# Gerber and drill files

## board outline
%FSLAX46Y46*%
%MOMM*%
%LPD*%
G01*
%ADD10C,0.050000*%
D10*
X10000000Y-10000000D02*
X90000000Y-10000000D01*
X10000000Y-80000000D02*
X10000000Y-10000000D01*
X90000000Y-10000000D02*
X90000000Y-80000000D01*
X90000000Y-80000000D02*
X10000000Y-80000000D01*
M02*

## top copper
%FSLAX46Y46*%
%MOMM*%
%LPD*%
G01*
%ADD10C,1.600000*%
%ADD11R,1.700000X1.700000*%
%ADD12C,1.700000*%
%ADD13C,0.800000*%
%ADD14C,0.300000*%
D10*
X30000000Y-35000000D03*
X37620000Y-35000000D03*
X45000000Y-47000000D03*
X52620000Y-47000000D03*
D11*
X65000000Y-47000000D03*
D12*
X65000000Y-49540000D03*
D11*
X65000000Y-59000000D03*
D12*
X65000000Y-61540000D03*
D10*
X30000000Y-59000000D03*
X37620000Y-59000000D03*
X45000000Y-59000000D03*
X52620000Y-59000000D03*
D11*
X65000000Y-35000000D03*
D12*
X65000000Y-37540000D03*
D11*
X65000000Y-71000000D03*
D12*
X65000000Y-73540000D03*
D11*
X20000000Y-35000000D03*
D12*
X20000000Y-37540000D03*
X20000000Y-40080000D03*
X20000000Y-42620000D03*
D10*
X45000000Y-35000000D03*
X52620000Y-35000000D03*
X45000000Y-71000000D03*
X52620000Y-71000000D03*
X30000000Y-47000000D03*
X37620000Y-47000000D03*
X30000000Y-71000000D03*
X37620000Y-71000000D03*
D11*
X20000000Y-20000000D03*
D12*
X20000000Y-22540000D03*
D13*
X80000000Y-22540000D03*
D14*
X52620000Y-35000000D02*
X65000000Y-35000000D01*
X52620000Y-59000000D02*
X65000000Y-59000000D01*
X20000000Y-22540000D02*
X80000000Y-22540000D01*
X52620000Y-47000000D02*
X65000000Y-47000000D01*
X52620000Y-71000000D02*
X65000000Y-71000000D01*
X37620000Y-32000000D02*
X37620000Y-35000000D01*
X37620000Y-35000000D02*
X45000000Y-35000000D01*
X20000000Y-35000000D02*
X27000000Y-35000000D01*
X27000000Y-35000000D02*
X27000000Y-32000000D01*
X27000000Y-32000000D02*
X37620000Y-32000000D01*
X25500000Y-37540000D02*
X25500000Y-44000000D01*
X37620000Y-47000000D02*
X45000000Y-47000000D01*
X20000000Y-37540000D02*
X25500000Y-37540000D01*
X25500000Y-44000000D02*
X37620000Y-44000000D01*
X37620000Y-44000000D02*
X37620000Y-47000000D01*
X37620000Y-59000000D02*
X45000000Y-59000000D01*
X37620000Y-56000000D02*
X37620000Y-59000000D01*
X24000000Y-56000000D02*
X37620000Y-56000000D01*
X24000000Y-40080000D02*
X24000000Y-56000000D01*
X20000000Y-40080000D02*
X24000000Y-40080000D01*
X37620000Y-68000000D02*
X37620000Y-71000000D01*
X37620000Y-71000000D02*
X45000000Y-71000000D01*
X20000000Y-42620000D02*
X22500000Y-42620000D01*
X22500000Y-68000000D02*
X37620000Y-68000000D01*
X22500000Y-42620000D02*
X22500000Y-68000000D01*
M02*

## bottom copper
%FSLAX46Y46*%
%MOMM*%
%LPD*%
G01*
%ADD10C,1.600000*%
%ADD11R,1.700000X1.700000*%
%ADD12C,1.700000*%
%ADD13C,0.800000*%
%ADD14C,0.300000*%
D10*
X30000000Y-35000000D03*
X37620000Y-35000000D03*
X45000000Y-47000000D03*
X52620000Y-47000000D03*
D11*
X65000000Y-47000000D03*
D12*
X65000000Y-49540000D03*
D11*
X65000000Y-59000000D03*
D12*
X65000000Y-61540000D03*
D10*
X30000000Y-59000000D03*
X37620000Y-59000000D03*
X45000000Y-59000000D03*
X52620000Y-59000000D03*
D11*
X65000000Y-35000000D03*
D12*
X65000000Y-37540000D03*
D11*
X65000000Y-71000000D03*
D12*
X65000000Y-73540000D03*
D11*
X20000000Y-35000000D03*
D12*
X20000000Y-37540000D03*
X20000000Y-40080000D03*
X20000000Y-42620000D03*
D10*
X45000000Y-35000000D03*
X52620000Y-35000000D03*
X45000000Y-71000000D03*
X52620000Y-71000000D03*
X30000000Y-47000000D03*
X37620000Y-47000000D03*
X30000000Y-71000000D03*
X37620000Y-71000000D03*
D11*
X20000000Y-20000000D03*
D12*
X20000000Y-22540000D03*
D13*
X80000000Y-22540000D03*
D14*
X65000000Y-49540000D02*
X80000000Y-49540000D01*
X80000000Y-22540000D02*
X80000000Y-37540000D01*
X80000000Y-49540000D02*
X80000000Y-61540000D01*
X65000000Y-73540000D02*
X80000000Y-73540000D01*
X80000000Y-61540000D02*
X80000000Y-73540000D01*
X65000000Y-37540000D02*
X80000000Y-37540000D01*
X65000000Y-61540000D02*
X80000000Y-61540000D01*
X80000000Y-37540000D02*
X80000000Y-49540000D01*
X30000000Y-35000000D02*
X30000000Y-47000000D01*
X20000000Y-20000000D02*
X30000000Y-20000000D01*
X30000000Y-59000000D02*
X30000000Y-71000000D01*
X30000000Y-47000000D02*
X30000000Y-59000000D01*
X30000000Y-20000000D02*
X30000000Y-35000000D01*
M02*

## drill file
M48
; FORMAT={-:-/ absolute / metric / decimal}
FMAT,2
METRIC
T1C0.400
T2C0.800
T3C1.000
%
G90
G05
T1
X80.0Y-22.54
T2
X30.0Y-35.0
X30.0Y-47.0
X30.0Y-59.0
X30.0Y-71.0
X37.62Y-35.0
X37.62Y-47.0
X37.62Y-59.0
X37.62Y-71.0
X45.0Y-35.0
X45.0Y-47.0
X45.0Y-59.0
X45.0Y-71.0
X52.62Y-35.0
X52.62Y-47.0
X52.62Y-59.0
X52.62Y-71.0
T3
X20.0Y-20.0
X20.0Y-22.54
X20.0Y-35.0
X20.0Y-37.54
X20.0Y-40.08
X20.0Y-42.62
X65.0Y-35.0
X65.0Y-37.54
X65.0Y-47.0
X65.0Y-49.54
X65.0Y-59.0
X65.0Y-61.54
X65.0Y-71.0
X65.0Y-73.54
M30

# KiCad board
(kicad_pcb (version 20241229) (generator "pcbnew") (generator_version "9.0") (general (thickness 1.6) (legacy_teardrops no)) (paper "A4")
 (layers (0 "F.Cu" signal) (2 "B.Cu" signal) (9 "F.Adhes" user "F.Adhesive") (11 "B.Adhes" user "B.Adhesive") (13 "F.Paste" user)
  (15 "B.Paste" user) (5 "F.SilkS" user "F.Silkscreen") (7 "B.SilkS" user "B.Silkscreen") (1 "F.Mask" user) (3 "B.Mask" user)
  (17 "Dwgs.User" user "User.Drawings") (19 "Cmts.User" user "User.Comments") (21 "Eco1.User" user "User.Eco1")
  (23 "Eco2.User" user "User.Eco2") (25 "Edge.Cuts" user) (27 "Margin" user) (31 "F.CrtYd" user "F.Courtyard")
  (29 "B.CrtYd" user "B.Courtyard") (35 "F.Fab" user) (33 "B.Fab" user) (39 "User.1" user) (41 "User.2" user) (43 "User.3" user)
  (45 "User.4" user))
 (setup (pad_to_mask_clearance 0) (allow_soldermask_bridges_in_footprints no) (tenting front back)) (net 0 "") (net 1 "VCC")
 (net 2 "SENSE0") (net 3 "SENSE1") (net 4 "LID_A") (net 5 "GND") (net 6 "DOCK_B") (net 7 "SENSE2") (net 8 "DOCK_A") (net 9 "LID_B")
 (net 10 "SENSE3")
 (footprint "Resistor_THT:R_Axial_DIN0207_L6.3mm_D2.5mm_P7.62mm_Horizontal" (layer "F.Cu") (at 30 35)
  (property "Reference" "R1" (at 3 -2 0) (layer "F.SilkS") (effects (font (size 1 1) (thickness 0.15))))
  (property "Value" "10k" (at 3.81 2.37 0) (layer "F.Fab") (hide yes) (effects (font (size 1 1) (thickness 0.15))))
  (pad "1" thru_hole circle (at 0 0) (size 1.6 1.6) (drill 0.8) (layers "*.Cu" "*.Mask") (remove_unused_layers no) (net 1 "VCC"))
  (pad "2" thru_hole circle (at 7.62 0) (size 1.6 1.6) (drill 0.8) (layers "*.Cu" "*.Mask") (remove_unused_layers no) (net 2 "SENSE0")))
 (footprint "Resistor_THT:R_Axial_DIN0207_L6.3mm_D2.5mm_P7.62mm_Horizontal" (layer "F.Cu") (at 45 47)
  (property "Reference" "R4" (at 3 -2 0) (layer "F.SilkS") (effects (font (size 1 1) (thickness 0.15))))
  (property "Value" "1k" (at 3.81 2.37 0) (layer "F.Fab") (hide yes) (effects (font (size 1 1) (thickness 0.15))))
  (pad "1" thru_hole circle (at 0 0) (size 1.6 1.6) (drill 0.8) (layers "*.Cu" "*.Mask") (remove_unused_layers no) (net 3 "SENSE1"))
  (pad "2" thru_hole circle (at 7.62 0) (size 1.6 1.6) (drill 0.8) (layers "*.Cu" "*.Mask") (remove_unused_layers no) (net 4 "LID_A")))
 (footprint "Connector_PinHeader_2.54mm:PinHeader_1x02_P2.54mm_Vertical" (layer "F.Cu") (at 65 47)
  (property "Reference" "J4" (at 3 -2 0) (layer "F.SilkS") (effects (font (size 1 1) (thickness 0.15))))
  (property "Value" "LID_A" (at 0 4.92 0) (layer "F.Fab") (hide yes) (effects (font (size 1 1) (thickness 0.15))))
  (pad "1" thru_hole rect (at 0 0) (size 1.7 1.7) (drill 1) (layers "*.Cu" "*.Mask") (remove_unused_layers no) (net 4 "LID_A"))
  (pad "2" thru_hole circle (at 0 2.54) (size 1.7 1.7) (drill 1) (layers "*.Cu" "*.Mask") (remove_unused_layers no) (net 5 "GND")))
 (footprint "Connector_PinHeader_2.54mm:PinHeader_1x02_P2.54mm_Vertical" (layer "F.Cu") (at 65 59)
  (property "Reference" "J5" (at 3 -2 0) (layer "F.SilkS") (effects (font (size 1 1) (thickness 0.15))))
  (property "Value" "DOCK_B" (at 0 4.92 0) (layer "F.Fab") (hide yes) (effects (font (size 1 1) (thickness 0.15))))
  (pad "1" thru_hole rect (at 0 0) (size 1.7 1.7) (drill 1) (layers "*.Cu" "*.Mask") (remove_unused_layers no) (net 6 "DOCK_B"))
  (pad "2" thru_hole circle (at 0 2.54) (size 1.7 1.7) (drill 1) (layers "*.Cu" "*.Mask") (remove_unused_layers no) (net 5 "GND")))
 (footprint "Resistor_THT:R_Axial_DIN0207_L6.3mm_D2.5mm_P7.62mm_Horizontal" (layer "F.Cu") (at 30 59)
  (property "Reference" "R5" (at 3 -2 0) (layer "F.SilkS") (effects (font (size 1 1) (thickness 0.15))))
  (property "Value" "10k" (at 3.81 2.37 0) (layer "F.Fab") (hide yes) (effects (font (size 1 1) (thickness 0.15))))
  (pad "1" thru_hole circle (at 0 0) (size 1.6 1.6) (drill 0.8) (layers "*.Cu" "*.Mask") (remove_unused_layers no) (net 1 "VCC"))
  (pad "2" thru_hole circle (at 7.62 0) (size 1.6 1.6) (drill 0.8) (layers "*.Cu" "*.Mask") (remove_unused_layers no) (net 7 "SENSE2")))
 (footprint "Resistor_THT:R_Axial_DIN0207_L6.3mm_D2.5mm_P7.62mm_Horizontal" (layer "F.Cu") (at 45 59)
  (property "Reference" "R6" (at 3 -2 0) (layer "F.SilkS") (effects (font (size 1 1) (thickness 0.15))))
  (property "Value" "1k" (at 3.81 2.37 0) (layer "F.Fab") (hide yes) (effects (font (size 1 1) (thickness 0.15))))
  (pad "1" thru_hole circle (at 0 0) (size 1.6 1.6) (drill 0.8) (layers "*.Cu" "*.Mask") (remove_unused_layers no) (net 7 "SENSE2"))
  (pad "2" thru_hole circle (at 7.62 0) (size 1.6 1.6) (drill 0.8) (layers "*.Cu" "*.Mask") (remove_unused_layers no) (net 6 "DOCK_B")))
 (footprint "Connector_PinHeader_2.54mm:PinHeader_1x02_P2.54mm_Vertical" (layer "F.Cu") (at 65 35)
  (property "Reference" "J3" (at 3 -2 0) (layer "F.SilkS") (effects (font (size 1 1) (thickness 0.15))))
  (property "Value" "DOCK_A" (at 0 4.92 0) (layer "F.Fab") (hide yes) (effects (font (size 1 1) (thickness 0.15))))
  (pad "1" thru_hole rect (at 0 0) (size 1.7 1.7) (drill 1) (layers "*.Cu" "*.Mask") (remove_unused_layers no) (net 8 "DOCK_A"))
  (pad "2" thru_hole circle (at 0 2.54) (size 1.7 1.7) (drill 1) (layers "*.Cu" "*.Mask") (remove_unused_layers no) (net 5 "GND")))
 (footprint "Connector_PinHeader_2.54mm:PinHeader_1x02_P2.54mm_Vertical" (layer "F.Cu") (at 65 71)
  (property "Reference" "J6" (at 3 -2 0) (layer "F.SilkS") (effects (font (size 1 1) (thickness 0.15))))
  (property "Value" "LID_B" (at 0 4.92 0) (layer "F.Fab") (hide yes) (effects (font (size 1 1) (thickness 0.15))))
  (pad "1" thru_hole rect (at 0 0) (size 1.7 1.7) (drill 1) (layers "*.Cu" "*.Mask") (remove_unused_layers no) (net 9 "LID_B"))
  (pad "2" thru_hole circle (at 0 2.54) (size 1.7 1.7) (drill 1) (layers "*.Cu" "*.Mask") (remove_unused_layers no) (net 5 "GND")))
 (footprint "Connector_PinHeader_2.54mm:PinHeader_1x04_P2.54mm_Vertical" (layer "F.Cu") (at 20 35)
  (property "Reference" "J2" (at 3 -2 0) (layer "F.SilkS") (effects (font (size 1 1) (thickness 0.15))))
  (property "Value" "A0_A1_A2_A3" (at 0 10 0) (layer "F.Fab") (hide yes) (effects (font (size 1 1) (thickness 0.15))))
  (pad "1" thru_hole rect (at 0 0) (size 1.7 1.7) (drill 1) (layers "*.Cu" "*.Mask") (remove_unused_layers no) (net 2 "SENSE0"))
  (pad "2" thru_hole circle (at 0 2.54) (size 1.7 1.7) (drill 1) (layers "*.Cu" "*.Mask") (remove_unused_layers no) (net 3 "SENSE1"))
  (pad "3" thru_hole circle (at 0 5.08) (size 1.7 1.7) (drill 1) (layers "*.Cu" "*.Mask") (remove_unused_layers no) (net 7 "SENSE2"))
  (pad "4" thru_hole circle (at 0 7.62) (size 1.7 1.7) (drill 1) (layers "*.Cu" "*.Mask") (remove_unused_layers no) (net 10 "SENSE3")))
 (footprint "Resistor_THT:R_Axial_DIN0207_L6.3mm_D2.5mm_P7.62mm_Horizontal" (layer "F.Cu") (at 45 35)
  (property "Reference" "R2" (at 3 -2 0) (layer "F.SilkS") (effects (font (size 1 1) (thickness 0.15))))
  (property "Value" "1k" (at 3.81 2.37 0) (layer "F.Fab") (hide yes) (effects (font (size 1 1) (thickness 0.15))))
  (pad "1" thru_hole circle (at 0 0) (size 1.6 1.6) (drill 0.8) (layers "*.Cu" "*.Mask") (remove_unused_layers no) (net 2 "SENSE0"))
  (pad "2" thru_hole circle (at 7.62 0) (size 1.6 1.6) (drill 0.8) (layers "*.Cu" "*.Mask") (remove_unused_layers no) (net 8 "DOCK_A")))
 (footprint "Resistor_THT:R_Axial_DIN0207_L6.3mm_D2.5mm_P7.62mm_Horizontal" (layer "F.Cu") (at 45 71)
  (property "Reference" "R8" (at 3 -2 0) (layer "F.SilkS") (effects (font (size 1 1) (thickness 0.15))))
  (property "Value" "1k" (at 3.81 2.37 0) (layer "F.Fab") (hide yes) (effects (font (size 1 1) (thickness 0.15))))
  (pad "1" thru_hole circle (at 0 0) (size 1.6 1.6) (drill 0.8) (layers "*.Cu" "*.Mask") (remove_unused_layers no) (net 10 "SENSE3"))
  (pad "2" thru_hole circle (at 7.62 0) (size 1.6 1.6) (drill 0.8) (layers "*.Cu" "*.Mask") (remove_unused_layers no) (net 9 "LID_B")))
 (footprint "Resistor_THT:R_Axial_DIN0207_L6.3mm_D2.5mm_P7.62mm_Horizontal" (layer "F.Cu") (at 30 47)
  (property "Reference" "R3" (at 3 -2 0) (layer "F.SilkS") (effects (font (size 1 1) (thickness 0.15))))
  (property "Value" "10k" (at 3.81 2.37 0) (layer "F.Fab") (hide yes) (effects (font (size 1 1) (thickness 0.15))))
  (pad "1" thru_hole circle (at 0 0) (size 1.6 1.6) (drill 0.8) (layers "*.Cu" "*.Mask") (remove_unused_layers no) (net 1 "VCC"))
  (pad "2" thru_hole circle (at 7.62 0) (size 1.6 1.6) (drill 0.8) (layers "*.Cu" "*.Mask") (remove_unused_layers no) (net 3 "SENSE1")))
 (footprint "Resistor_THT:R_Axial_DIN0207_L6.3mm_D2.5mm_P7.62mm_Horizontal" (layer "F.Cu") (at 30 71)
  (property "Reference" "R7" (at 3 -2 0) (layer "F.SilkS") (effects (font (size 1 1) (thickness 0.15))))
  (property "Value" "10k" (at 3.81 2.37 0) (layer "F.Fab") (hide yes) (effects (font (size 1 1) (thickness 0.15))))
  (pad "1" thru_hole circle (at 0 0) (size 1.6 1.6) (drill 0.8) (layers "*.Cu" "*.Mask") (remove_unused_layers no) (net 1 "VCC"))
  (pad "2" thru_hole circle (at 7.62 0) (size 1.6 1.6) (drill 0.8) (layers "*.Cu" "*.Mask") (remove_unused_layers no) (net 10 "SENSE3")))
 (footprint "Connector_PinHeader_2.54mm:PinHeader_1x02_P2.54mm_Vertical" (layer "F.Cu") (at 20 20)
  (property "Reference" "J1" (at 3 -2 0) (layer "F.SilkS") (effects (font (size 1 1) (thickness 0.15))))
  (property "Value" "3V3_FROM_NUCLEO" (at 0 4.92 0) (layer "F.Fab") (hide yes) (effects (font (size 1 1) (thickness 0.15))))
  (pad "1" thru_hole rect (at 0 0) (size 1.7 1.7) (drill 1) (layers "*.Cu" "*.Mask") (remove_unused_layers no) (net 1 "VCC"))
  (pad "2" thru_hole circle (at 0 2.54) (size 1.7 1.7) (drill 1) (layers "*.Cu" "*.Mask") (remove_unused_layers no) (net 5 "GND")))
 (gr_line (start 10 10) (end 90 10) (stroke (width 0.05) (type default)) (layer "Edge.Cuts"))
 (gr_line (start 10 80) (end 10 10) (stroke (width 0.05) (type default)) (layer "Edge.Cuts"))
 (gr_line (start 90 10) (end 90 80) (stroke (width 0.05) (type default)) (layer "Edge.Cuts"))
 (gr_line (start 90 80) (end 10 80) (stroke (width 0.05) (type default)) (layer "Edge.Cuts"))
 (segment (start 52.62 35) (end 65 35) (width 0.3) (layer "F.Cu") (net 8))
 (segment (start 52.62 59) (end 65 59) (width 0.3) (layer "F.Cu") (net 6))
 (segment (start 20 22.54) (end 80 22.54) (width 0.3) (layer "F.Cu") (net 5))
 (via (at 80 22.54) (size 0.8) (drill 0.4) (layers "F.Cu" "B.Cu") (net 5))
 (segment (start 65 49.54) (end 80 49.54) (width 0.3) (layer "B.Cu") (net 5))
 (segment (start 80 22.54) (end 80 37.54) (width 0.3) (layer "B.Cu") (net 5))
 (segment (start 80 49.54) (end 80 61.54) (width 0.3) (layer "B.Cu") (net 5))
 (segment (start 65 73.54) (end 80 73.54) (width 0.3) (layer "B.Cu") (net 5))
 (segment (start 80 61.54) (end 80 73.54) (width 0.3) (layer "B.Cu") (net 5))
 (segment (start 65 37.54) (end 80 37.54) (width 0.3) (layer "B.Cu") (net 5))
 (segment (start 65 61.54) (end 80 61.54) (width 0.3) (layer "B.Cu") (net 5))
 (segment (start 80 37.54) (end 80 49.54) (width 0.3) (layer "B.Cu") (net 5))
 (segment (start 52.62 47) (end 65 47) (width 0.3) (layer "F.Cu") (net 4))
 (segment (start 52.62 71) (end 65 71) (width 0.3) (layer "F.Cu") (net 9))
 (segment (start 37.62 32) (end 37.62 35) (width 0.3) (layer "F.Cu") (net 2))
 (segment (start 37.62 35) (end 45 35) (width 0.3) (layer "F.Cu") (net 2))
 (segment (start 20 35) (end 27 35) (width 0.3) (layer "F.Cu") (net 2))
 (segment (start 27 35) (end 27 32) (width 0.3) (layer "F.Cu") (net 2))
 (segment (start 27 32) (end 37.62 32) (width 0.3) (layer "F.Cu") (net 2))
 (segment (start 25.5 37.54) (end 25.5 44) (width 0.3) (layer "F.Cu") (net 3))
 (segment (start 37.62 47) (end 45 47) (width 0.3) (layer "F.Cu") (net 3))
 (segment (start 20 37.54) (end 25.5 37.54) (width 0.3) (layer "F.Cu") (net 3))
 (segment (start 25.5 44) (end 37.62 44) (width 0.3) (layer "F.Cu") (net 3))
 (segment (start 37.62 44) (end 37.62 47) (width 0.3) (layer "F.Cu") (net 3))
 (segment (start 37.62 59) (end 45 59) (width 0.3) (layer "F.Cu") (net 7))
 (segment (start 37.62 56) (end 37.62 59) (width 0.3) (layer "F.Cu") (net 7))
 (segment (start 24 56) (end 37.62 56) (width 0.3) (layer "F.Cu") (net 7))
 (segment (start 24 40.08) (end 24 56) (width 0.3) (layer "F.Cu") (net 7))
 (segment (start 20 40.08) (end 24 40.08) (width 0.3) (layer "F.Cu") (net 7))
 (segment (start 37.62 68) (end 37.62 71) (width 0.3) (layer "F.Cu") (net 10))
 (segment (start 37.62 71) (end 45 71) (width 0.3) (layer "F.Cu") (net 10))
 (segment (start 20 42.62) (end 22.5 42.62) (width 0.3) (layer "F.Cu") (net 10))
 (segment (start 22.5 68) (end 37.62 68) (width 0.3) (layer "F.Cu") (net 10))
 (segment (start 22.5 42.62) (end 22.5 68) (width 0.3) (layer "F.Cu") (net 10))
 (segment (start 30 35) (end 30 47) (width 0.3) (layer "B.Cu") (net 1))
 (segment (start 20 20) (end 30 20) (width 0.3) (layer "B.Cu") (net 1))
 (segment (start 30 59) (end 30 71) (width 0.3) (layer "B.Cu") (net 1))
 (segment (start 30 47) (end 30 59) (width 0.3) (layer "B.Cu") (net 1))
 (segment (start 30 20) (end 30 35) (width 0.3) (layer "B.Cu") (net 1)))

